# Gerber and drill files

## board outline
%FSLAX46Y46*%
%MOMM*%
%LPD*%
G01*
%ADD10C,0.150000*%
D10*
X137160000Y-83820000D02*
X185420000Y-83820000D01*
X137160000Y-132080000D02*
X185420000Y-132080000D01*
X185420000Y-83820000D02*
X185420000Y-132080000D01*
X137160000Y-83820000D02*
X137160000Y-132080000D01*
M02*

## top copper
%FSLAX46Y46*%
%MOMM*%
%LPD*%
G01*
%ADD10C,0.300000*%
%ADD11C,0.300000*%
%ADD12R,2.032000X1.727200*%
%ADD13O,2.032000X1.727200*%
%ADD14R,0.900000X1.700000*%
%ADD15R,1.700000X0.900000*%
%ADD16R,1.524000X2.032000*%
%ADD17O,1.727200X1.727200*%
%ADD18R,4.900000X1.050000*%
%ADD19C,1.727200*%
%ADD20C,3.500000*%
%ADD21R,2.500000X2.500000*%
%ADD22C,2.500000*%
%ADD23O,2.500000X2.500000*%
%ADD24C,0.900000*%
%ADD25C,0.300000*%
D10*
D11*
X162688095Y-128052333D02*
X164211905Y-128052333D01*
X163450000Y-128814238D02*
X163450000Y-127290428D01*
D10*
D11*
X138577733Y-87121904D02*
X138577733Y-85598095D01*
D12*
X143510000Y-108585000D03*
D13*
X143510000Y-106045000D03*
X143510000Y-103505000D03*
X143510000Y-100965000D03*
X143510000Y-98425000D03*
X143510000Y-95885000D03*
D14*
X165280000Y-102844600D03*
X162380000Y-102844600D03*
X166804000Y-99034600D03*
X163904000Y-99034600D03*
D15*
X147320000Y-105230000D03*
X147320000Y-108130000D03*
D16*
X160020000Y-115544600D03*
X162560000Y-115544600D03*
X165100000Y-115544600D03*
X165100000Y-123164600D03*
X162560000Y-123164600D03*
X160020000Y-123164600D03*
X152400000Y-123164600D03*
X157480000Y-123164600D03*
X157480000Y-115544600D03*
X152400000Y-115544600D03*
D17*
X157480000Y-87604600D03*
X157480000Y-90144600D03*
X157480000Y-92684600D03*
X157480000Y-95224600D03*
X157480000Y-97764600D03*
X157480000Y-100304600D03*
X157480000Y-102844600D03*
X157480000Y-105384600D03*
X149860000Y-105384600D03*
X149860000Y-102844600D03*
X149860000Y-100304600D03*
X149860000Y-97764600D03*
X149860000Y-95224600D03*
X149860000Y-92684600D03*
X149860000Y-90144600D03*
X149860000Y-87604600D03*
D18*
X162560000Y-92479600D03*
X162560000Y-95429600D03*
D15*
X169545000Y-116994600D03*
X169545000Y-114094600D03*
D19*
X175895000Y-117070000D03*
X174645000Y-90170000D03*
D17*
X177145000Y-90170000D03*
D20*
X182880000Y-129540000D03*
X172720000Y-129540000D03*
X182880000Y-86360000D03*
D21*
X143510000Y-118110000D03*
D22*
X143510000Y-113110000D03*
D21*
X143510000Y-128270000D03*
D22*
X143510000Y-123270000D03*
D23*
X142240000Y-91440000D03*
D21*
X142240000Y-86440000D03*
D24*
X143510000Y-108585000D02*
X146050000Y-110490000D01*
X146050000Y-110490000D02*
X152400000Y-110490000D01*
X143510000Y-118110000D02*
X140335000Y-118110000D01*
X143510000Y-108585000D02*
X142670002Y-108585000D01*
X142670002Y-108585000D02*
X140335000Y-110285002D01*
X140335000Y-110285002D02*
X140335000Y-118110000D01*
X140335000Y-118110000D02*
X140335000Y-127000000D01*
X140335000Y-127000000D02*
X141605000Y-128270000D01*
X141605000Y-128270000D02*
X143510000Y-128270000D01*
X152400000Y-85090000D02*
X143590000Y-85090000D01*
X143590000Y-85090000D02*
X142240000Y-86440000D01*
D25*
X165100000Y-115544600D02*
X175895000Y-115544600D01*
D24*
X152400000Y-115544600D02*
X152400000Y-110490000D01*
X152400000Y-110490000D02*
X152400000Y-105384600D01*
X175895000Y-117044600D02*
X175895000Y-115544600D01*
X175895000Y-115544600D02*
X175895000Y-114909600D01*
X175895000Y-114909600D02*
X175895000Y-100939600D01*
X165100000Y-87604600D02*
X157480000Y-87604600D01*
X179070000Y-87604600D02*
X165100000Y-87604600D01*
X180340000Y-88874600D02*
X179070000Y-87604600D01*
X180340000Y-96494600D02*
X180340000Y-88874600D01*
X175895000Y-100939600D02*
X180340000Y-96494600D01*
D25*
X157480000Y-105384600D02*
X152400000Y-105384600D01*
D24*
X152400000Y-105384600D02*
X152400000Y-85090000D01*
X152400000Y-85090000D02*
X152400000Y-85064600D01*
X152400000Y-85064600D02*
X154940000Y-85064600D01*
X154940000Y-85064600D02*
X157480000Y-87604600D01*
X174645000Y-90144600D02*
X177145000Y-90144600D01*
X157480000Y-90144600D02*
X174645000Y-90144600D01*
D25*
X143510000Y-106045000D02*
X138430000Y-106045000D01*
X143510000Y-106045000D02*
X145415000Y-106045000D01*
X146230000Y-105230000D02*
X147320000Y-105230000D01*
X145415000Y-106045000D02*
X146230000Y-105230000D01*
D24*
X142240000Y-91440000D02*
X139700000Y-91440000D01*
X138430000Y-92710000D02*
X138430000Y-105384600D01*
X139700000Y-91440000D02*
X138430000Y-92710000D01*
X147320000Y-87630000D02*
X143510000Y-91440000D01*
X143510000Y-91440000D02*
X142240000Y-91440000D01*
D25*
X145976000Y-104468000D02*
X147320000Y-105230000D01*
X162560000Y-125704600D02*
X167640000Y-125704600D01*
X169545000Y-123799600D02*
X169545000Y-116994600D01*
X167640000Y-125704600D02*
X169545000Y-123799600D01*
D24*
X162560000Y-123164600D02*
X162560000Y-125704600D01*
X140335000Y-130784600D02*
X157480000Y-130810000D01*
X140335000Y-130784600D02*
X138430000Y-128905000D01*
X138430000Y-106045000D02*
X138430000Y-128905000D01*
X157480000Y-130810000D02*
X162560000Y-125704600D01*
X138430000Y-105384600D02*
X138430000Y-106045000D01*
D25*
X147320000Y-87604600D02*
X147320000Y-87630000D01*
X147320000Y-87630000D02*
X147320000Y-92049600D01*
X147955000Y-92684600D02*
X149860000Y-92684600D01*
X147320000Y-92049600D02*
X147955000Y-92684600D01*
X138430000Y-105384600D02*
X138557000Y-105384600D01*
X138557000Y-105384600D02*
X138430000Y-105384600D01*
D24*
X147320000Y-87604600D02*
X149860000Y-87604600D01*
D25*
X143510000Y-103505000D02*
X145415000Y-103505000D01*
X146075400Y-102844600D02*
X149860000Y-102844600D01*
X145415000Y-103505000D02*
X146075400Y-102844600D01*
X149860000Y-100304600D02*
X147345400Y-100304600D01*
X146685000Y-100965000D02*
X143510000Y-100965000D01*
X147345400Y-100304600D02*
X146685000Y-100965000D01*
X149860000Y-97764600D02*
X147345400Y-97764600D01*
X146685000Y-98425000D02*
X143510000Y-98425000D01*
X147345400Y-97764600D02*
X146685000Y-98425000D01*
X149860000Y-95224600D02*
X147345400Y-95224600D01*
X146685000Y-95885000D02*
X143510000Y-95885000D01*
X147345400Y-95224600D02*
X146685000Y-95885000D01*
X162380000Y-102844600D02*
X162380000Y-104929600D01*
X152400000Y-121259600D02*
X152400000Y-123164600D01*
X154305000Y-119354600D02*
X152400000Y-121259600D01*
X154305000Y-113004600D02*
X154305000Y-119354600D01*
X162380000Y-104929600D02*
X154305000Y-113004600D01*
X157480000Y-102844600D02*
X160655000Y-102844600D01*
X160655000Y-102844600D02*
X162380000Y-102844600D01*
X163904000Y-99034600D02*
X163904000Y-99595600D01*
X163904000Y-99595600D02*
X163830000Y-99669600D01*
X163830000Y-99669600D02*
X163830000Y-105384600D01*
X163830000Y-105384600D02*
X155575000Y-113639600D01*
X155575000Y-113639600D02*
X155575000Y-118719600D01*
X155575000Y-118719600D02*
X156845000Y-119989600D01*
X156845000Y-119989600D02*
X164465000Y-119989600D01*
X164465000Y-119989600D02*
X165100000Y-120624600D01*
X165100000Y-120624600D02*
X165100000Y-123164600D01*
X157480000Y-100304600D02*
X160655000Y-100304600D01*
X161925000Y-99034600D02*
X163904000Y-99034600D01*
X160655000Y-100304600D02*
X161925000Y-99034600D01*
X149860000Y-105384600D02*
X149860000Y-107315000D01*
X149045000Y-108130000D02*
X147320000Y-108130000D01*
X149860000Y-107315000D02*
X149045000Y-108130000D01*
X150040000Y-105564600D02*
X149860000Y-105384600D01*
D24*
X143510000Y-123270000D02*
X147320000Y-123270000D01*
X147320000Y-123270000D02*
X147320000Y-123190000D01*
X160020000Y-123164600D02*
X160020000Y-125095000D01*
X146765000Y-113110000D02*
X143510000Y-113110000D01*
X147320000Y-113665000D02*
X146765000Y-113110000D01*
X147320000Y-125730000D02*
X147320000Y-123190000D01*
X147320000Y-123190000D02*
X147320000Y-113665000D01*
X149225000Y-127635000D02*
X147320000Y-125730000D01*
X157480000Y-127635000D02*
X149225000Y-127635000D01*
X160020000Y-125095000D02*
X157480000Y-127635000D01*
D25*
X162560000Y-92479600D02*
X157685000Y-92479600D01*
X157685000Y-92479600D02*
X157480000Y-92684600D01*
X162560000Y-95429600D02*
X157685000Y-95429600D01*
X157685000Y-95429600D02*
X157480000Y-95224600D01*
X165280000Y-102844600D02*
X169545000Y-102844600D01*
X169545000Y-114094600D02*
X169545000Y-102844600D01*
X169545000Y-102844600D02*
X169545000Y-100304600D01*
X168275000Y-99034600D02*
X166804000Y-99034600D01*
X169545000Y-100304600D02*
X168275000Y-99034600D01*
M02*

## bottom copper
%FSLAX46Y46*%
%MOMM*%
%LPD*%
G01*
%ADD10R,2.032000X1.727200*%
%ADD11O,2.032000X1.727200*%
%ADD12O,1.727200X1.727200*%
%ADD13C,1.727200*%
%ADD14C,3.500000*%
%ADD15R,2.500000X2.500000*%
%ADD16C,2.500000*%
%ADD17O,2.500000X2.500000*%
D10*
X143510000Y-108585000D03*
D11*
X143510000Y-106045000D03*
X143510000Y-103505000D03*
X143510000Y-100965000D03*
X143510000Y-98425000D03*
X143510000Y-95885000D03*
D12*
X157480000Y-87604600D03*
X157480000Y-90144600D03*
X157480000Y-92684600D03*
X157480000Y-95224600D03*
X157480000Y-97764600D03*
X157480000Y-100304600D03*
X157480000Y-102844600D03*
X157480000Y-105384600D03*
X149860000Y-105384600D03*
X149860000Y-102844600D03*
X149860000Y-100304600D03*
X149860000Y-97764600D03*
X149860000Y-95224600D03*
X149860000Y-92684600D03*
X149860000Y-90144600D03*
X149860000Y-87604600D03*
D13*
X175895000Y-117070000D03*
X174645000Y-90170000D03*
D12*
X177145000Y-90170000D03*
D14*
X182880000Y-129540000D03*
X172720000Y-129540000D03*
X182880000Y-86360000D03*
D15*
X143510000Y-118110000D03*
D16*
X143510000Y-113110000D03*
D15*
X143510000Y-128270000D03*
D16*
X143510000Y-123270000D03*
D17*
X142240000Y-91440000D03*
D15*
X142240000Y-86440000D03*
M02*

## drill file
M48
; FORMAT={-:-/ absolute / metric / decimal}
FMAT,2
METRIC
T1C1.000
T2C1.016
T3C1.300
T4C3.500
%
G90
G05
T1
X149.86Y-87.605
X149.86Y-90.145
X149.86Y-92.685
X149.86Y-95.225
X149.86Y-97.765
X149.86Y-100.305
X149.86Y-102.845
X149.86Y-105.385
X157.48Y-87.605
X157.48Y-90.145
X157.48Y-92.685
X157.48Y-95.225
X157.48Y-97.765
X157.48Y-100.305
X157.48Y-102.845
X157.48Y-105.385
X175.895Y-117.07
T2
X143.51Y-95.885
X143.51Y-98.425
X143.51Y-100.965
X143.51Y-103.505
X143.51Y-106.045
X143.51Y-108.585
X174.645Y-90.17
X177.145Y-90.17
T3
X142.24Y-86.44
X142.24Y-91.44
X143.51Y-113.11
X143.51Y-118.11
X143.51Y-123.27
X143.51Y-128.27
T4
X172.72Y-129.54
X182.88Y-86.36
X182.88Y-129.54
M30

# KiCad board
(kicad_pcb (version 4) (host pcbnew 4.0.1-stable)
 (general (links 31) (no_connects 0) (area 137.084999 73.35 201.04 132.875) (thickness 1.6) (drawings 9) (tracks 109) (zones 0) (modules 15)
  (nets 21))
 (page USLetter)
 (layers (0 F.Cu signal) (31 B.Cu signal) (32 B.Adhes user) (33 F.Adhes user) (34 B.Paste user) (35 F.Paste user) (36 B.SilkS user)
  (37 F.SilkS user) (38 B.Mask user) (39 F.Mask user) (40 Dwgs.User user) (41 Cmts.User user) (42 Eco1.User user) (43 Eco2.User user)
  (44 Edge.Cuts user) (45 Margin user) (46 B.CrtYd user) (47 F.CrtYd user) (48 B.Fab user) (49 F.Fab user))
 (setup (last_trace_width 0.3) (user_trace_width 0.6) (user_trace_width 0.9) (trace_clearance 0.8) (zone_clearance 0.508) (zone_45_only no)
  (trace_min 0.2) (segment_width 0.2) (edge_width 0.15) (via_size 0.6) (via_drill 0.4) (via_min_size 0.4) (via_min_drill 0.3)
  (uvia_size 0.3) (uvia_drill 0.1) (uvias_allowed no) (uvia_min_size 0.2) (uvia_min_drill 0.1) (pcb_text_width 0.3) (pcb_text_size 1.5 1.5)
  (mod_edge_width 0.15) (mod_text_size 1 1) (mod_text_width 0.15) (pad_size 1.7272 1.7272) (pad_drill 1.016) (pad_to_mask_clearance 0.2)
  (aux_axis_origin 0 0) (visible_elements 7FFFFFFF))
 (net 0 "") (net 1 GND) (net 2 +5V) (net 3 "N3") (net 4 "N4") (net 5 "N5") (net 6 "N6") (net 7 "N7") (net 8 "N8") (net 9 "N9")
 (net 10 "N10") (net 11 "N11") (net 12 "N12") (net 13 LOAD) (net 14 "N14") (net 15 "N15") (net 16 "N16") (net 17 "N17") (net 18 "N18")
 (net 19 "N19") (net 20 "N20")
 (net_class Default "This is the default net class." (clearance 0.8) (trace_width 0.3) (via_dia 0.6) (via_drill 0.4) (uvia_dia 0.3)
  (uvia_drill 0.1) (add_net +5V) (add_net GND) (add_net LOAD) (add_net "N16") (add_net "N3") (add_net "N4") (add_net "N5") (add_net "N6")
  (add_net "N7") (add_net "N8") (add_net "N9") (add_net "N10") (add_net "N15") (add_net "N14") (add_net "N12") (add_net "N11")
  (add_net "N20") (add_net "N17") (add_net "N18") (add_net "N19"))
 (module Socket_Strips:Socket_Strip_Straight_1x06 (layer B.Cu) (at 143.51 108.585 90)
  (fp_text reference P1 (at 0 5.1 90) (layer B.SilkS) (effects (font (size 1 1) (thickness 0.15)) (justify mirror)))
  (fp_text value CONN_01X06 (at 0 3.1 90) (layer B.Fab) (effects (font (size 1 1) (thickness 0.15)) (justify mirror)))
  (pad 1 thru_hole rect (at 0 0 90) (size 1.7272 2.032) (drill 1.016) (layers *.Cu *.Mask B.SilkS) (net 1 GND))
  (pad 2 thru_hole oval (at 2.54 0 90) (size 1.7272 2.032) (drill 1.016) (layers *.Cu *.Mask B.SilkS) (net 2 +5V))
  (pad 3 thru_hole oval (at 5.08 0 90) (size 1.7272 2.032) (drill 1.016) (layers *.Cu *.Mask B.SilkS) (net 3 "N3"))
  (pad 4 thru_hole oval (at 7.62 0 90) (size 1.7272 2.032) (drill 1.016) (layers *.Cu *.Mask B.SilkS) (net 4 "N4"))
  (pad 5 thru_hole oval (at 10.16 0 90) (size 1.7272 2.032) (drill 1.016) (layers *.Cu *.Mask B.SilkS) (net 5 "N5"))
  (pad 6 thru_hole oval (at 12.7 0 90) (size 1.7272 2.032) (drill 1.016) (layers *.Cu *.Mask B.SilkS) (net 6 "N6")))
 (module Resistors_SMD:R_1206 (layer F.Cu) (at 163.83 102.8446 180)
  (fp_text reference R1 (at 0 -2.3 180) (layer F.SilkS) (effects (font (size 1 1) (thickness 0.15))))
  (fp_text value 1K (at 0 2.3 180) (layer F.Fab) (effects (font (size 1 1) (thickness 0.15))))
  (pad 1 smd rect (at -1.45 0 180) (size 0.9 1.7) (layers F.Cu F.Paste F.Mask) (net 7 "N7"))
  (pad 2 smd rect (at 1.45 0 180) (size 0.9 1.7) (layers F.Cu F.Paste F.Mask) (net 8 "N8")))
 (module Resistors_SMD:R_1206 (layer F.Cu) (at 165.354 99.0346 180)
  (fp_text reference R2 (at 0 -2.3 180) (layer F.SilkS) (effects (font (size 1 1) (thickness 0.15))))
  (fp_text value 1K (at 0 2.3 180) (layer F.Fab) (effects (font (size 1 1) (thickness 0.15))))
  (pad 1 smd rect (at -1.45 0 180) (size 0.9 1.7) (layers F.Cu F.Paste F.Mask) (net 7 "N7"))
  (pad 2 smd rect (at 1.45 0 180) (size 0.9 1.7) (layers F.Cu F.Paste F.Mask) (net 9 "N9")))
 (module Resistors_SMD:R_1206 (layer F.Cu) (at 147.32 106.68 270)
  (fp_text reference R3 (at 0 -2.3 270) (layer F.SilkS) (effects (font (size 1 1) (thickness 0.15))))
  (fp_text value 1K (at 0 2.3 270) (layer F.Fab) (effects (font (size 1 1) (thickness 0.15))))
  (pad 1 smd rect (at -1.45 0 270) (size 0.9 1.7) (layers F.Cu F.Paste F.Mask) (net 2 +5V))
  (pad 2 smd rect (at 1.45 0 270) (size 0.9 1.7) (layers F.Cu F.Paste F.Mask) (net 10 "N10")))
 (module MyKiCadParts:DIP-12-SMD (layer F.Cu) (at 152.4 123.1646)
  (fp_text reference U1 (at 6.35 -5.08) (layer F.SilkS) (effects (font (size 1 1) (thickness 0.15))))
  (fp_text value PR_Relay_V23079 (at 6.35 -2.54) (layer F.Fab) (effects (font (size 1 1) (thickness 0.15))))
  (pad 9 smd rect (at 7.62 -7.62) (size 1.524 2.032) (layers F.Cu F.Paste F.Mask) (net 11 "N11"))
  (pad 8 smd rect (at 10.16 -7.62) (size 1.524 2.032) (layers F.Cu F.Paste F.Mask) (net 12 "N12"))
  (pad 7 smd rect (at 12.7 -7.62) (size 1.524 2.032) (layers F.Cu F.Paste F.Mask) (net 1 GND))
  (pad 6 smd rect (at 12.7 0) (size 1.524 2.032) (layers F.Cu F.Paste F.Mask) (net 9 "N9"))
  (pad 5 smd rect (at 10.16 0) (size 1.524 2.032) (layers F.Cu F.Paste F.Mask) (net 2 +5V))
  (pad 4 smd rect (at 7.62 0) (size 1.524 2.032) (layers F.Cu F.Paste F.Mask) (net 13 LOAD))
  (pad 1 smd rect (at 0 0) (size 1.524 2.032) (layers F.Cu F.Paste F.Mask) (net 8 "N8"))
  (pad 3 smd rect (at 5.08 0) (size 1.524 2.032) (layers F.Cu F.Paste F.Mask) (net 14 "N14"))
  (pad 10 smd rect (at 5.08 -7.62) (size 1.524 2.032) (layers F.Cu F.Paste F.Mask) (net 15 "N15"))
  (pad 12 smd rect (at 0 -7.62) (size 1.524 2.032) (layers F.Cu F.Paste F.Mask) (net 1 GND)))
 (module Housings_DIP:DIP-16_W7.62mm (layer B.Cu) (at 157.48 87.6046 180)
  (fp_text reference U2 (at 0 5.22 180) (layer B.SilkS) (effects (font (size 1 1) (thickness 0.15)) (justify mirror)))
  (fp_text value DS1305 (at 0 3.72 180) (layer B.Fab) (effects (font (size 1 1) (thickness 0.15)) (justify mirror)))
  (pad 1 thru_hole oval (at 0 0 180) (size 1.7272 1.7272) (drill 1) (layers *.Cu *.Mask B.SilkS) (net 1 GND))
  (pad 2 thru_hole oval (at 0 -2.54 180) (size 1.7272 1.7272) (drill 1) (layers *.Cu *.Mask B.SilkS) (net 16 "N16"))
  (pad 3 thru_hole oval (at 0 -5.08 180) (size 1.7272 1.7272) (drill 1) (layers *.Cu *.Mask B.SilkS) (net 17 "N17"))
  (pad 4 thru_hole oval (at 0 -7.62 180) (size 1.7272 1.7272) (drill 1) (layers *.Cu *.Mask B.SilkS) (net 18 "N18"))
  (pad 5 thru_hole oval (at 0 -10.16 180) (size 1.7272 1.7272) (drill 1) (layers *.Cu *.Mask B.SilkS) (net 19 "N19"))
  (pad 6 thru_hole oval (at 0 -12.7 180) (size 1.7272 1.7272) (drill 1) (layers *.Cu *.Mask B.SilkS) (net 9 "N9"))
  (pad 7 thru_hole oval (at 0 -15.24 180) (size 1.7272 1.7272) (drill 1) (layers *.Cu *.Mask B.SilkS) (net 8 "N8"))
  (pad 8 thru_hole oval (at 0 -17.78 180) (size 1.7272 1.7272) (drill 1) (layers *.Cu *.Mask B.SilkS) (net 1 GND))
  (pad 9 thru_hole oval (at 7.62 -17.78 180) (size 1.7272 1.7272) (drill 1) (layers *.Cu *.Mask B.SilkS) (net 10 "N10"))
  (pad 10 thru_hole oval (at 7.62 -15.24 180) (size 1.7272 1.7272) (drill 1) (layers *.Cu *.Mask B.SilkS) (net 3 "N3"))
  (pad 11 thru_hole oval (at 7.62 -12.7 180) (size 1.7272 1.7272) (drill 1) (layers *.Cu *.Mask B.SilkS) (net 4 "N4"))
  (pad 12 thru_hole oval (at 7.62 -10.16 180) (size 1.7272 1.7272) (drill 1) (layers *.Cu *.Mask B.SilkS) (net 5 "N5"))
  (pad 13 thru_hole oval (at 7.62 -7.62 180) (size 1.7272 1.7272) (drill 1) (layers *.Cu *.Mask B.SilkS) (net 6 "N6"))
  (pad 14 thru_hole oval (at 7.62 -5.08 180) (size 1.7272 1.7272) (drill 1) (layers *.Cu *.Mask B.SilkS) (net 2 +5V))
  (pad 15 thru_hole oval (at 7.62 -2.54 180) (size 1.7272 1.7272) (drill 1) (layers *.Cu *.Mask B.SilkS) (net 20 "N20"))
  (pad 16 thru_hole oval (at 7.62 0 180) (size 1.7272 1.7272) (drill 1) (layers *.Cu *.Mask B.SilkS) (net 2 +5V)))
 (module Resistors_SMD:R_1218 (layer F.Cu) (at 162.56 93.9546 270)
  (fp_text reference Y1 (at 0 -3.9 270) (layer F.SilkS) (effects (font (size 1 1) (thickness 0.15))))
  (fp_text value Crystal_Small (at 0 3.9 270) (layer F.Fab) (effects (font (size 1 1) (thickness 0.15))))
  (pad 1 smd rect (at -1.475 0 270) (size 1.05 4.9) (layers F.Cu F.Paste F.Mask) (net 17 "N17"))
  (pad 2 smd rect (at 1.475 0 270) (size 1.05 4.9) (layers F.Cu F.Paste F.Mask) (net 18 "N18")))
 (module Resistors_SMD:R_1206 (layer F.Cu) (at 169.545 115.5446 90)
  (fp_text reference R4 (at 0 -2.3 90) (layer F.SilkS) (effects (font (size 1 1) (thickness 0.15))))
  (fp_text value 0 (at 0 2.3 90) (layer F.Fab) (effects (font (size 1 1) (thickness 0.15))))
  (pad 1 smd rect (at -1.45 0 90) (size 0.9 1.7) (layers F.Cu F.Paste F.Mask) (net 2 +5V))
  (pad 2 smd rect (at 1.45 0 90) (size 0.9 1.7) (layers F.Cu F.Paste F.Mask) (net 7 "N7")))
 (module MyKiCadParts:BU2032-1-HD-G (layer B.Cu) (at 175.895 90.17 270)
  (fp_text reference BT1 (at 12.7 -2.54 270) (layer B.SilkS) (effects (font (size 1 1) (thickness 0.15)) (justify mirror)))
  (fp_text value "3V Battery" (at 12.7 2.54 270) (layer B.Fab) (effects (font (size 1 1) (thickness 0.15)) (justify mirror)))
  (pad 2 thru_hole circle (at 26.9 0 270) (size 1.7272 1.7272) (drill 1) (layers *.Cu *.Mask B.SilkS) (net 1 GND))
  (pad 1 thru_hole circle (at 0 1.25 270) (size 1.7272 1.7272) (drill 1.016) (layers *.Cu *.Mask B.SilkS) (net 16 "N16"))
  (pad 1 thru_hole oval (at 0 -1.25 270) (size 1.7272 1.7272) (drill 1.016) (layers *.Cu *.Mask B.SilkS) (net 16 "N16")))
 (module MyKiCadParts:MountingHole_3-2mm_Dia (layer F.Cu) (at 182.88 129.54)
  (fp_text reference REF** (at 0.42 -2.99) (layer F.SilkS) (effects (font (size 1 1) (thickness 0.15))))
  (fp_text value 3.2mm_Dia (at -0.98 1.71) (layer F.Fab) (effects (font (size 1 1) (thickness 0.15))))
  (pad 1 thru_hole circle (at 0 0) (size 3.5 3.5) (drill 3.5) (layers)))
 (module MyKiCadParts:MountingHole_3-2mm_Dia (layer F.Cu) (at 172.72 129.54)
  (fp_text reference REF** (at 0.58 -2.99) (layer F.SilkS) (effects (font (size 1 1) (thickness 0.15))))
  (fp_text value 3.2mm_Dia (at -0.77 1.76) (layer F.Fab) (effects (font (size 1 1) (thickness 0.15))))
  (pad 1 thru_hole circle (at 0 0) (size 3.5 3.5) (drill 3.5) (layers)))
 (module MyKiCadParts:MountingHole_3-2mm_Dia (layer F.Cu) (at 182.88 86.36)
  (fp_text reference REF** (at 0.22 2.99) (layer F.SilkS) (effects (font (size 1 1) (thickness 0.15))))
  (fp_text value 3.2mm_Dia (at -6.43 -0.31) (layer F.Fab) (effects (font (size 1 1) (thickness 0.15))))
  (pad 1 thru_hole circle (at 0 0) (size 3.5 3.5) (drill 3.5) (layers)))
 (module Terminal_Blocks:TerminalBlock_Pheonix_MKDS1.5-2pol (layer B.Cu) (at 143.51 118.11 90)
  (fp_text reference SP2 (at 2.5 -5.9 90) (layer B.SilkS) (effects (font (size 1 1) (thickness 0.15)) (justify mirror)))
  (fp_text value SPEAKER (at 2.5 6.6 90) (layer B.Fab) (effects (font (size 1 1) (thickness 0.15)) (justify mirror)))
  (pad 1 thru_hole rect (at 0 0 90) (size 2.5 2.5) (drill 1.3) (layers *.Cu *.Mask B.SilkS) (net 1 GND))
  (pad 2 thru_hole circle (at 5 0 90) (size 2.5 2.5) (drill 1.3) (layers *.Cu *.Mask B.SilkS) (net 13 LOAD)))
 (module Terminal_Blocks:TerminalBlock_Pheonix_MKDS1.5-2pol (layer B.Cu) (at 143.51 128.27 90)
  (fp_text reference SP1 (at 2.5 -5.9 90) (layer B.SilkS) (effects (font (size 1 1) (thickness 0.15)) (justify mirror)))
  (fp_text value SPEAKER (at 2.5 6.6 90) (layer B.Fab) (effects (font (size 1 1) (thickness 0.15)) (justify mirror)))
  (pad 1 thru_hole rect (at 0 0 90) (size 2.5 2.5) (drill 1.3) (layers *.Cu *.Mask B.SilkS) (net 1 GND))
  (pad 2 thru_hole circle (at 5 0 90) (size 2.5 2.5) (drill 1.3) (layers *.Cu *.Mask B.SilkS) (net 13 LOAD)))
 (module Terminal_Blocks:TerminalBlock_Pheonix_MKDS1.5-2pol (layer B.Cu) (at 142.24 91.44 90)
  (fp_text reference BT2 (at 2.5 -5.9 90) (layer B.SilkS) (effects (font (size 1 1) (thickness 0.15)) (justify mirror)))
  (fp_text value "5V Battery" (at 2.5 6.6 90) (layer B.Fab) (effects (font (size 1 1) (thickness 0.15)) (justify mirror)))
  (pad 1 thru_hole oval (at 0 0 90) (size 2.5 2.5) (drill 1.3) (layers *.Cu *.Mask B.SilkS) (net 2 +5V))
  (pad 2 thru_hole rect (at 5 0 90) (size 2.5 2.5) (drill 1.3) (layers *.Cu *.Mask B.SilkS) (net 1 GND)))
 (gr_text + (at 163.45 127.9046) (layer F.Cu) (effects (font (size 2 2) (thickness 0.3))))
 (gr_line (start 137.16 83.82) (end 185.42 83.82) (angle 90) (layer Edge.Cuts) (width 0.15))
 (gr_line (start 137.16 132.08) (end 185.42 132.08) (angle 90) (layer Edge.Cuts) (width 0.15))
 (gr_line (start 185.42 83.82) (end 185.42 132.08) (angle 90) (layer Edge.Cuts) (width 0.15))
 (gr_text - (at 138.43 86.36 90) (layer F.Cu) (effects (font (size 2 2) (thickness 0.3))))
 (gr_line (start 137.16 83.82) (end 137.16 132.08) (angle 90) (layer Edge.Cuts) (width 0.15))
 (segment (start 143.51 108.585) (end 146.05 110.49) (width 0.9) (layer F.Cu) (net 1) (status 10))
 (segment (start 146.05 110.49) (end 152.4 110.49) (width 0.9) (layer F.Cu) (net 1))
 (segment (start 143.51 118.11) (end 140.335 118.11) (width 0.9) (layer F.Cu) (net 1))
 (segment (start 143.51 108.585) (end 142.670002 108.585) (width 0.9) (layer F.Cu) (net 1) (status 30))
 (segment (start 142.670002 108.585) (end 140.335 110.285002) (width 0.9) (layer F.Cu) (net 1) (status 10))
 (segment (start 140.335 110.285002) (end 140.335 118.11) (width 0.9) (layer F.Cu) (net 1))
 (segment (start 140.335 118.11) (end 140.335 127) (width 0.9) (layer F.Cu) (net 1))
 (segment (start 140.335 127) (end 141.605 128.27) (width 0.9) (layer F.Cu) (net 1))
 (segment (start 141.605 128.27) (end 143.51 128.27) (width 0.9) (layer F.Cu) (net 1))
 (segment (start 152.4 85.09) (end 143.59 85.09) (width 0.9) (layer F.Cu) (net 1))
 (segment (start 143.59 85.09) (end 142.24 86.44) (width 0.9) (layer F.Cu) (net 1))
 (segment (start 165.1 115.5446) (end 175.895 115.5446) (width 0.3) (layer F.Cu) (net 1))
 (segment (start 152.4 115.5446) (end 152.4 110.49) (width 0.9) (layer F.Cu) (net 1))
 (segment (start 152.4 110.49) (end 152.4 105.3846) (width 0.9) (layer F.Cu) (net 1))
 (segment (start 175.895 117.0446) (end 175.895 115.5446) (width 0.9) (layer F.Cu) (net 1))
 (segment (start 175.895 115.5446) (end 175.895 114.9096) (width 0.9) (layer F.Cu) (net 1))
 (segment (start 175.895 114.9096) (end 175.895 100.9396) (width 0.9) (layer F.Cu) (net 1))
 (segment (start 165.1 87.6046) (end 157.48 87.6046) (width 0.9) (layer F.Cu) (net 1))
 (segment (start 179.07 87.6046) (end 165.1 87.6046) (width 0.9) (layer F.Cu) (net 1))
 (segment (start 180.34 88.8746) (end 179.07 87.6046) (width 0.9) (layer F.Cu) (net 1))
 (segment (start 180.34 96.4946) (end 180.34 88.8746) (width 0.9) (layer F.Cu) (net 1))
 (segment (start 175.895 100.9396) (end 180.34 96.4946) (width 0.9) (layer F.Cu) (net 1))
 (segment (start 157.48 105.3846) (end 152.4 105.3846) (width 0.3) (layer F.Cu) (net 1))
 (segment (start 152.4 105.3846) (end 152.4 85.09) (width 0.9) (layer F.Cu) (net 1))
 (segment (start 152.4 85.09) (end 152.4 85.0646) (width 0.9) (layer F.Cu) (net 1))
 (segment (start 152.4 85.0646) (end 154.94 85.0646) (width 0.9) (layer F.Cu) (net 1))
 (segment (start 154.94 85.0646) (end 157.48 87.6046) (width 0.9) (layer F.Cu) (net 1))
 (segment (start 174.645 90.1446) (end 177.145 90.1446) (width 0.9) (layer F.Cu) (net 16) (status 30))
 (segment (start 157.48 90.1446) (end 174.645 90.1446) (width 0.9) (layer F.Cu) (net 16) (status 20))
 (segment (start 143.51 106.045) (end 138.43 106.045) (width 0.3) (layer F.Cu) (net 2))
 (segment (start 143.51 106.045) (end 145.415 106.045) (width 0.3) (layer F.Cu) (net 2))
 (segment (start 146.23 105.23) (end 147.32 105.23) (width 0.3) (layer F.Cu) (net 2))
 (segment (start 145.415 106.045) (end 146.23 105.23) (width 0.3) (layer F.Cu) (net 2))
 (segment (start 142.24 91.44) (end 139.7 91.44) (width 0.9) (layer F.Cu) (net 2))
 (segment (start 138.43 92.71) (end 138.43 105.3846) (width 0.9) (layer F.Cu) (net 2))
 (segment (start 139.7 91.44) (end 138.43 92.71) (width 0.9) (layer F.Cu) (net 2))
 (segment (start 147.32 87.63) (end 143.51 91.44) (width 0.9) (layer F.Cu) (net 2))
 (segment (start 143.51 91.44) (end 142.24 91.44) (width 0.9) (layer F.Cu) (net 2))
 (segment (start 145.976 104.468) (end 147.32 105.23) (width 0.3) (layer F.Cu) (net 2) (status 20))
 (segment (start 162.56 125.7046) (end 167.64 125.7046) (width 0.3) (layer F.Cu) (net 2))
 (segment (start 169.545 123.7996) (end 169.545 116.9946) (width 0.3) (layer F.Cu) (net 2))
 (segment (start 167.64 125.7046) (end 169.545 123.7996) (width 0.3) (layer F.Cu) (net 2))
 (segment (start 162.56 123.1646) (end 162.56 125.7046) (width 0.9) (layer F.Cu) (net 2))
 (segment (start 140.335 130.7846) (end 157.48 130.81) (width 0.9) (layer F.Cu) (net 2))
 (segment (start 140.335 130.7846) (end 138.43 128.905) (width 0.9) (layer F.Cu) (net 2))
 (segment (start 138.43 106.045) (end 138.43 128.905) (width 0.9) (layer F.Cu) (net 2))
 (segment (start 157.48 130.81) (end 162.56 125.7046) (width 0.9) (layer F.Cu) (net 2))
 (segment (start 138.43 105.3846) (end 138.43 106.045) (width 0.9) (layer F.Cu) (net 2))
 (segment (start 147.32 87.6046) (end 147.32 87.63) (width 0.3) (layer F.Cu) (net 2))
 (segment (start 147.32 87.63) (end 147.32 92.0496) (width 0.3) (layer F.Cu) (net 2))
 (segment (start 147.955 92.6846) (end 149.86 92.6846) (width 0.3) (layer F.Cu) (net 2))
 (segment (start 147.32 92.0496) (end 147.955 92.6846) (width 0.3) (layer F.Cu) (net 2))
 (segment (start 138.43 105.3846) (end 138.557 105.3846) (width 0.3) (layer F.Cu) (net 2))
 (segment (start 138.557 105.3846) (end 138.43 105.3846) (width 0.3) (layer F.Cu) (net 2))
 (segment (start 147.32 87.6046) (end 149.86 87.6046) (width 0.9) (layer F.Cu) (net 2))
 (segment (start 143.51 103.505) (end 145.415 103.505) (width 0.3) (layer F.Cu) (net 3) (status 400000))
 (segment (start 146.0754 102.8446) (end 149.86 102.8446) (width 0.3) (layer F.Cu) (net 3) (status 800000))
 (segment (start 145.415 103.505) (end 146.0754 102.8446) (width 0.3) (layer F.Cu) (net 3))
 (segment (start 149.86 100.3046) (end 147.3454 100.3046) (width 0.3) (layer F.Cu) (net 4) (status 400000))
 (segment (start 146.685 100.965) (end 143.51 100.965) (width 0.3) (layer F.Cu) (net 4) (status 800000))
 (segment (start 147.3454 100.3046) (end 146.685 100.965) (width 0.3) (layer F.Cu) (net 4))
 (segment (start 149.86 97.7646) (end 147.3454 97.7646) (width 0.3) (layer F.Cu) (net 5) (status 400000))
 (segment (start 146.685 98.425) (end 143.51 98.425) (width 0.3) (layer F.Cu) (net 5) (status 800000))
 (segment (start 147.3454 97.7646) (end 146.685 98.425) (width 0.3) (layer F.Cu) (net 5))
 (segment (start 149.86 95.2246) (end 147.3454 95.2246) (width 0.3) (layer F.Cu) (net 6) (status 400000))
 (segment (start 146.685 95.885) (end 143.51 95.885) (width 0.3) (layer F.Cu) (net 6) (status 800000))
 (segment (start 147.3454 95.2246) (end 146.685 95.885) (width 0.3) (layer F.Cu) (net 6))
 (segment (start 162.38 102.8446) (end 162.38 104.9296) (width 0.3) (layer F.Cu) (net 8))
 (segment (start 152.4 121.2596) (end 152.4 123.1646) (width 0.3) (layer F.Cu) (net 8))
 (segment (start 154.305 119.3546) (end 152.4 121.2596) (width 0.3) (layer F.Cu) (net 8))
 (segment (start 154.305 113.0046) (end 154.305 119.3546) (width 0.3) (layer F.Cu) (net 8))
 (segment (start 162.38 104.9296) (end 154.305 113.0046) (width 0.3) (layer F.Cu) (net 8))
 (segment (start 157.48 102.8446) (end 160.655 102.8446) (width 0.3) (layer F.Cu) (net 8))
 (segment (start 160.655 102.8446) (end 162.38 102.8446) (width 0.3) (layer F.Cu) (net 8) (status 20))
 (segment (start 163.904 99.0346) (end 163.904 99.5956) (width 0.3) (layer F.Cu) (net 9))
 (segment (start 163.904 99.5956) (end 163.83 99.6696) (width 0.3) (layer F.Cu) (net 9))
 (segment (start 163.83 99.6696) (end 163.83 105.3846) (width 0.3) (layer F.Cu) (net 9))
 (segment (start 163.83 105.3846) (end 155.575 113.6396) (width 0.3) (layer F.Cu) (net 9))
 (segment (start 155.575 113.6396) (end 155.575 118.7196) (width 0.3) (layer F.Cu) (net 9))
 (segment (start 155.575 118.7196) (end 156.845 119.9896) (width 0.3) (layer F.Cu) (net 9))
 (segment (start 156.845 119.9896) (end 164.465 119.9896) (width 0.3) (layer F.Cu) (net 9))
 (segment (start 164.465 119.9896) (end 165.1 120.6246) (width 0.3) (layer F.Cu) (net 9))
 (segment (start 165.1 120.6246) (end 165.1 123.1646) (width 0.3) (layer F.Cu) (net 9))
 (segment (start 157.48 100.3046) (end 160.655 100.3046) (width 0.3) (layer F.Cu) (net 9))
 (segment (start 161.925 99.0346) (end 163.904 99.0346) (width 0.3) (layer F.Cu) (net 9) (status 20))
 (segment (start 160.655 100.3046) (end 161.925 99.0346) (width 0.3) (layer F.Cu) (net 9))
 (segment (start 149.86 105.3846) (end 149.86 107.315) (width 0.3) (layer F.Cu) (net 10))
 (segment (start 149.045 108.13) (end 147.32 108.13) (width 0.3) (layer F.Cu) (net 10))
 (segment (start 149.86 107.315) (end 149.045 108.13) (width 0.3) (layer F.Cu) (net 10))
 (segment (start 150.04 105.5646) (end 149.86 105.3846) (width 0.3) (layer F.Cu) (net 10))
 (segment (start 143.51 123.27) (end 147.32 123.27) (width 0.9) (layer F.Cu) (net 13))
 (segment (start 147.32 123.27) (end 147.32 123.19) (width 0.9) (layer F.Cu) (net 13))
 (segment (start 160.02 123.1646) (end 160.02 125.095) (width 0.9) (layer F.Cu) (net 13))
 (segment (start 146.765 113.11) (end 143.51 113.11) (width 0.9) (layer F.Cu) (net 13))
 (segment (start 147.32 113.665) (end 146.765 113.11) (width 0.9) (layer F.Cu) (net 13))
 (segment (start 147.32 125.73) (end 147.32 123.19) (width 0.9) (layer F.Cu) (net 13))
 (segment (start 147.32 123.19) (end 147.32 113.665) (width 0.9) (layer F.Cu) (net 13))
 (segment (start 149.225 127.635) (end 147.32 125.73) (width 0.9) (layer F.Cu) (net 13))
 (segment (start 157.48 127.635) (end 149.225 127.635) (width 0.9) (layer F.Cu) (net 13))
 (segment (start 160.02 125.095) (end 157.48 127.635) (width 0.9) (layer F.Cu) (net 13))
 (segment (start 162.56 92.4796) (end 157.685 92.4796) (width 0.3) (layer F.Cu) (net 17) (status 10))
 (segment (start 157.685 92.4796) (end 157.48 92.6846) (width 0.3) (layer F.Cu) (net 17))
 (segment (start 162.56 95.4296) (end 157.685 95.4296) (width 0.3) (layer F.Cu) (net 18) (status 10))
 (segment (start 157.685 95.4296) (end 157.48 95.2246) (width 0.3) (layer F.Cu) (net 18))
 (segment (start 165.28 102.8446) (end 169.545 102.8446) (width 0.3) (layer F.Cu) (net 7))
 (segment (start 169.545 114.0946) (end 169.545 102.8446) (width 0.3) (layer F.Cu) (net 7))
 (segment (start 169.545 102.8446) (end 169.545 100.3046) (width 0.3) (layer F.Cu) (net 7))
 (segment (start 168.275 99.0346) (end 166.804 99.0346) (width 0.3) (layer F.Cu) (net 7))
 (segment (start 169.545 100.3046) (end 168.275 99.0346) (width 0.3) (layer F.Cu) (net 7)))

